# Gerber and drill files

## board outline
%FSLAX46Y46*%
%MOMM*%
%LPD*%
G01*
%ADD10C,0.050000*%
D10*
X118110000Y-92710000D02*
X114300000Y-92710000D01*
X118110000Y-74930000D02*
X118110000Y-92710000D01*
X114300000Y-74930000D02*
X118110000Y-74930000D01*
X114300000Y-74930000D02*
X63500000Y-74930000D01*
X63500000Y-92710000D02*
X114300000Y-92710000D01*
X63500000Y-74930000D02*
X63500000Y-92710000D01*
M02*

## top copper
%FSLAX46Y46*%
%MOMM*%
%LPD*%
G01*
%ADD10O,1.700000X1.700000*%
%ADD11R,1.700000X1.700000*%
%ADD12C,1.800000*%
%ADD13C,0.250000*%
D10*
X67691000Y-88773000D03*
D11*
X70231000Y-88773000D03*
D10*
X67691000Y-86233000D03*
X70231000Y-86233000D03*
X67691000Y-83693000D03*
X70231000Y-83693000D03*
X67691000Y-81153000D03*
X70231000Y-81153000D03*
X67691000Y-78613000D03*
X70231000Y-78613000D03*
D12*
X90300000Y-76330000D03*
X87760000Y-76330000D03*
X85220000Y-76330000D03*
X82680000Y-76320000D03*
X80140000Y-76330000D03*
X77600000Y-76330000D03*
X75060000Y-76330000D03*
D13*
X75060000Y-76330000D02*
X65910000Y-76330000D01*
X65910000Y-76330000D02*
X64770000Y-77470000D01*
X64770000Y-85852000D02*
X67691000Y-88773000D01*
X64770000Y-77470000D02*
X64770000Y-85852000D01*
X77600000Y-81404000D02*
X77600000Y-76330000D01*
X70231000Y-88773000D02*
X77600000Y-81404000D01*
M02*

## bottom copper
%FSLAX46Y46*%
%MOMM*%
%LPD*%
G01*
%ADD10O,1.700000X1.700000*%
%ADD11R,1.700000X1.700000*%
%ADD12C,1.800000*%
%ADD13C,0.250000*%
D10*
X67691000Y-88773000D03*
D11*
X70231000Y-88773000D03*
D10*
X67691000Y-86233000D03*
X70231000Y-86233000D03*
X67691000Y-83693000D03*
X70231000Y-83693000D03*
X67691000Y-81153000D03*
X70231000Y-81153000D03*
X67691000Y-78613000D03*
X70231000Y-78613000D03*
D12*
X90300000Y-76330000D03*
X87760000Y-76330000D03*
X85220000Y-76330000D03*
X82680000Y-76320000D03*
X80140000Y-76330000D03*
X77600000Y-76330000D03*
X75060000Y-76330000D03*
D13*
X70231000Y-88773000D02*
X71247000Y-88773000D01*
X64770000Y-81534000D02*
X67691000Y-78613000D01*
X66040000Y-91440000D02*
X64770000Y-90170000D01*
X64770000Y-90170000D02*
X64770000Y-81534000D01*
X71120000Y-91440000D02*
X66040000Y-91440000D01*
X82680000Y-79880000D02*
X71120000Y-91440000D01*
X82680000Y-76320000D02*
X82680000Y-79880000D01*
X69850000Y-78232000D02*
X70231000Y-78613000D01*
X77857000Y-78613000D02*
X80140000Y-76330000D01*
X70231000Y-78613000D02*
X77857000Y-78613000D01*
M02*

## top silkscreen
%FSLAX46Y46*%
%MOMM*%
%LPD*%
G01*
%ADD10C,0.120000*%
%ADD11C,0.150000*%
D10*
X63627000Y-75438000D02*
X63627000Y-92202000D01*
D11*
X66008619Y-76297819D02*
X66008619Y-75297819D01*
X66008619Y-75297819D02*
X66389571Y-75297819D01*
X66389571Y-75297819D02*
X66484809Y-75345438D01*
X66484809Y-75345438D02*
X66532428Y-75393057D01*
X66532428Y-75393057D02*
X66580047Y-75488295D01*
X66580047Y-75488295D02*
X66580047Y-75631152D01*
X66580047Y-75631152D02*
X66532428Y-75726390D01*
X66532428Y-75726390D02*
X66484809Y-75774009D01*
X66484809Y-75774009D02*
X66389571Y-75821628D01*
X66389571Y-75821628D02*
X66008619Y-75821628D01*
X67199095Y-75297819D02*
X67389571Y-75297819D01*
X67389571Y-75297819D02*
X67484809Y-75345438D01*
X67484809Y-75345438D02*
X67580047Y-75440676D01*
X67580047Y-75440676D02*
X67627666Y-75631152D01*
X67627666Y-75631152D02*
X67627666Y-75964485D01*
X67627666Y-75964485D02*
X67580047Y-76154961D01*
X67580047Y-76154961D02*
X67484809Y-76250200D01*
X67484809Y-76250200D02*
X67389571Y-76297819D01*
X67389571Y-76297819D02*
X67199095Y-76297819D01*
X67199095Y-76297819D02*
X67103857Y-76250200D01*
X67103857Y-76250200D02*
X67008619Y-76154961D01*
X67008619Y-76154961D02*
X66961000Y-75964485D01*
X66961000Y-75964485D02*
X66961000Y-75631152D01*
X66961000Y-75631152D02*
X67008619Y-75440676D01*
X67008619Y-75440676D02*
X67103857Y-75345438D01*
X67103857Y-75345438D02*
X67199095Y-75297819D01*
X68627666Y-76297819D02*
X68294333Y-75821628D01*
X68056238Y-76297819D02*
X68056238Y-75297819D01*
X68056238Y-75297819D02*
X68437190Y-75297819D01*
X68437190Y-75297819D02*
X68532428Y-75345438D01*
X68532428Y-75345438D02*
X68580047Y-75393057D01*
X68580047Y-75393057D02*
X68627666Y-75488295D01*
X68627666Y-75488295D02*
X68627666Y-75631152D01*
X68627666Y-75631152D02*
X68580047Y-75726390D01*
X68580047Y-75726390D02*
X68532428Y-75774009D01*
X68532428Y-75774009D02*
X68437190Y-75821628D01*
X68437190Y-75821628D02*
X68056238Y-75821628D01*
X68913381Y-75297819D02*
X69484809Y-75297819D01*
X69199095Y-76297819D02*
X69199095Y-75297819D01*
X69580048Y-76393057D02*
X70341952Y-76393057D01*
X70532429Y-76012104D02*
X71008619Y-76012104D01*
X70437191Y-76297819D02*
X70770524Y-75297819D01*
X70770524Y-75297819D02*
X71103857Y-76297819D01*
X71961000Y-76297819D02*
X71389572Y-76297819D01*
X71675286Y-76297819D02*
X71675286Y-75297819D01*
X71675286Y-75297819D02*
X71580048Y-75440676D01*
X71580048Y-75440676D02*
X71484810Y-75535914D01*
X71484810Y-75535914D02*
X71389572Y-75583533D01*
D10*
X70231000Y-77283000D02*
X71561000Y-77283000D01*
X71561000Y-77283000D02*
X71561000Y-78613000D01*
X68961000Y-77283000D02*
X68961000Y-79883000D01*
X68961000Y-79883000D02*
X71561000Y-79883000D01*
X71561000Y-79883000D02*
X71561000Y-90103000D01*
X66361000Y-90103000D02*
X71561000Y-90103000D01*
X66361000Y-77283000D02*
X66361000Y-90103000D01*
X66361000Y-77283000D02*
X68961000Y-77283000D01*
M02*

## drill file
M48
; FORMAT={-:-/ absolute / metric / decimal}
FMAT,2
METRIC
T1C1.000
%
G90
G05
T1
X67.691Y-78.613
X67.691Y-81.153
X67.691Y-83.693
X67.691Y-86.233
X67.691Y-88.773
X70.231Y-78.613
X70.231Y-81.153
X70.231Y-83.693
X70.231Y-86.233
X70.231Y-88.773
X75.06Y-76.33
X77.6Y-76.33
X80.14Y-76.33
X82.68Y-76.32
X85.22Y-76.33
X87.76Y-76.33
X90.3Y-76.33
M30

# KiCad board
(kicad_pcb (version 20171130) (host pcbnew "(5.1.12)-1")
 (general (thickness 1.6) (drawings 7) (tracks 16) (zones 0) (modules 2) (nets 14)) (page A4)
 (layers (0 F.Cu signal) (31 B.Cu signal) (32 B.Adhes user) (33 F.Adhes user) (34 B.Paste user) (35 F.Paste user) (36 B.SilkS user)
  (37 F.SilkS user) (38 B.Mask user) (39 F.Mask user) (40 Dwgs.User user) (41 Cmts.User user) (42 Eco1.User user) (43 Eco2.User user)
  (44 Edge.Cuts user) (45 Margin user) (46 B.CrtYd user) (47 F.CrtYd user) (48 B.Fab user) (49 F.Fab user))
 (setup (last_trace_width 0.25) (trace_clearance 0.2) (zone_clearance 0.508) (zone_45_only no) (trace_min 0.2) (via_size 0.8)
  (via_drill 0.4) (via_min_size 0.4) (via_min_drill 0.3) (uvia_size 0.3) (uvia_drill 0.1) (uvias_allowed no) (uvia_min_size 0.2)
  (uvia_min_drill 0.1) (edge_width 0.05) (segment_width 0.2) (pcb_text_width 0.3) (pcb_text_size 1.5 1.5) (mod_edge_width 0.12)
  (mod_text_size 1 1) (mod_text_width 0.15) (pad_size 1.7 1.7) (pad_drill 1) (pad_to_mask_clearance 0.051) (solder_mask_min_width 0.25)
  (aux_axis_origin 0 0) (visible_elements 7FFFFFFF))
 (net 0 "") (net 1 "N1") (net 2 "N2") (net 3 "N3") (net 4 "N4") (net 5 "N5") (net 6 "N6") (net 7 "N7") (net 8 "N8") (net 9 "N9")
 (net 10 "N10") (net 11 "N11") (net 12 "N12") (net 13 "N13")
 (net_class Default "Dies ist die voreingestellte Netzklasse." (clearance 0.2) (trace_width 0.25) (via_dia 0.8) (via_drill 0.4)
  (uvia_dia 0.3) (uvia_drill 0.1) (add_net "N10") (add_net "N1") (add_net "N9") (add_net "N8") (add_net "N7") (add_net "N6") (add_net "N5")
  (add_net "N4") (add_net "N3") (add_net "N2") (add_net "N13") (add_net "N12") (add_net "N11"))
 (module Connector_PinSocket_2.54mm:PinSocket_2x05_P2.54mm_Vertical (layer F.Cu) (at 70.231 78.613)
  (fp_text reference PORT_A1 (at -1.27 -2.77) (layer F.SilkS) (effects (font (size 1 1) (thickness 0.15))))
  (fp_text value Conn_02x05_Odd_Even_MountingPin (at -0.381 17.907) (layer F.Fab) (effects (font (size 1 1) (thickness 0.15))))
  (fp_line (start 0 -1.33) (end 1.33 -1.33) (layer F.SilkS) (width 0.12))
  (fp_line (start 1.33 -1.33) (end 1.33 0) (layer F.SilkS) (width 0.12))
  (fp_line (start -1.27 -1.33) (end -1.27 1.27) (layer F.SilkS) (width 0.12))
  (fp_line (start -1.27 1.27) (end 1.33 1.27) (layer F.SilkS) (width 0.12))
  (fp_line (start 1.33 1.27) (end 1.33 11.49) (layer F.SilkS) (width 0.12))
  (fp_line (start -3.87 11.49) (end 1.33 11.49) (layer F.SilkS) (width 0.12))
  (fp_line (start -3.87 -1.33) (end -3.87 11.49) (layer F.SilkS) (width 0.12))
  (fp_line (start -3.87 -1.33) (end -1.27 -1.33) (layer F.SilkS) (width 0.12))
  (pad 10 thru_hole oval (at -2.54 10.16) (size 1.7 1.7) (drill 1) (layers *.Cu *.Mask) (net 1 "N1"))
  (pad 9 thru_hole rect (at 0 10.16) (size 1.7 1.7) (drill 1) (layers *.Cu *.Mask) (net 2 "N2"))
  (pad 8 thru_hole oval (at -2.54 7.62) (size 1.7 1.7) (drill 1) (layers *.Cu *.Mask) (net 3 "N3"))
  (pad 7 thru_hole oval (at 0 7.62) (size 1.7 1.7) (drill 1) (layers *.Cu *.Mask) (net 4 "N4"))
  (pad 6 thru_hole oval (at -2.54 5.08) (size 1.7 1.7) (drill 1) (layers *.Cu *.Mask) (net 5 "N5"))
  (pad 5 thru_hole oval (at 0 5.08) (size 1.7 1.7) (drill 1) (layers *.Cu *.Mask) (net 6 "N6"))
  (pad 4 thru_hole oval (at -2.54 2.54) (size 1.7 1.7) (drill 1) (layers *.Cu *.Mask) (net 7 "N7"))
  (pad 3 thru_hole oval (at 0 2.54) (size 1.7 1.7) (drill 1) (layers *.Cu *.Mask) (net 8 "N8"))
  (pad 2 thru_hole oval (at -2.54 0) (size 1.7 1.7) (drill 1) (layers *.Cu *.Mask) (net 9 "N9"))
  (pad 1 thru_hole oval (at 0 0) (size 1.7 1.7) (drill 1) (layers *.Cu *.Mask) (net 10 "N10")))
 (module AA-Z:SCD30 (layer F.Cu) (at 73.66 74.93 180)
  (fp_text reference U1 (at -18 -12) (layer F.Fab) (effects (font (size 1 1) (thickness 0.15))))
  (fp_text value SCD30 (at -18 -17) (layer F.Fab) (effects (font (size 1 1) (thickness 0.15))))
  (pad 7 thru_hole circle (at -16.64 -1.4 180) (size 1.8 1.8) (drill 1) (layers *.Cu *.Mask) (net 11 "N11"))
  (pad 6 thru_hole circle (at -14.1 -1.4 180) (size 1.8 1.8) (drill 1) (layers *.Cu *.Mask) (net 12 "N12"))
  (pad 5 thru_hole circle (at -11.56 -1.4 180) (size 1.8 1.8) (drill 1) (layers *.Cu *.Mask) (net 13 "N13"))
  (pad 4 thru_hole circle (at -9.02 -1.39 180) (size 1.8 1.8) (drill 1) (layers *.Cu *.Mask) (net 9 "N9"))
  (pad 3 thru_hole circle (at -6.48 -1.4 180) (size 1.8 1.8) (drill 1) (layers *.Cu *.Mask) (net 10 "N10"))
  (pad 2 thru_hole circle (at -3.94 -1.4 180) (size 1.8 1.8) (drill 1) (layers *.Cu *.Mask) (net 2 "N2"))
  (pad 1 thru_hole circle (at -1.4 -1.4 180) (size 1.8 1.8) (drill 1) (layers *.Cu *.Mask) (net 1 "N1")))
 (gr_line (start 118.11 92.71) (end 114.3 92.71) (layer Edge.Cuts) (width 0.05))
 (gr_line (start 118.11 74.93) (end 118.11 92.71) (layer Edge.Cuts) (width 0.05))
 (gr_line (start 114.3 74.93) (end 118.11 74.93) (layer Edge.Cuts) (width 0.05))
 (gr_line (start 114.3 74.93) (end 63.5 74.93) (layer Edge.Cuts) (width 0.05))
 (gr_line (start 63.5 92.71) (end 114.3 92.71) (layer Edge.Cuts) (width 0.05))
 (gr_line (start 63.5 74.93) (end 63.5 92.71) (layer Edge.Cuts) (width 0.05))
 (gr_line (start 63.627 75.438) (end 63.627 92.202) (layer F.SilkS) (width 0.12))
 (segment (start 75.06 76.33) (end 65.91 76.33) (width 0.25) (layer F.Cu) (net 1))
 (segment (start 65.91 76.33) (end 64.77 77.47) (width 0.25) (layer F.Cu) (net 1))
 (segment (start 64.77 85.852) (end 67.691 88.773) (width 0.25) (layer F.Cu) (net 1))
 (segment (start 64.77 77.47) (end 64.77 85.852) (width 0.25) (layer F.Cu) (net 1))
 (segment (start 70.231 88.773) (end 71.247 88.773) (width 0.25) (layer B.Cu) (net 2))
 (segment (start 77.6 81.404) (end 77.6 76.33) (width 0.25) (layer F.Cu) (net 2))
 (segment (start 70.231 88.773) (end 77.6 81.404) (width 0.25) (layer F.Cu) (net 2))
 (segment (start 64.77 81.534) (end 67.691 78.613) (width 0.25) (layer B.Cu) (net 9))
 (segment (start 66.04 91.44) (end 64.77 90.17) (width 0.25) (layer B.Cu) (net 9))
 (segment (start 64.77 90.17) (end 64.77 81.534) (width 0.25) (layer B.Cu) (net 9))
 (segment (start 71.12 91.44) (end 66.04 91.44) (width 0.25) (layer B.Cu) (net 9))
 (segment (start 82.68 79.88) (end 71.12 91.44) (width 0.25) (layer B.Cu) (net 9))
 (segment (start 82.68 76.32) (end 82.68 79.88) (width 0.25) (layer B.Cu) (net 9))
 (segment (start 69.85 78.232) (end 70.231 78.613) (width 0.25) (layer B.Cu) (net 10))
 (segment (start 77.857 78.613) (end 80.14 76.33) (width 0.25) (layer B.Cu) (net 10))
 (segment (start 70.231 78.613) (end 77.857 78.613) (width 0.25) (layer B.Cu) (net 10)))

